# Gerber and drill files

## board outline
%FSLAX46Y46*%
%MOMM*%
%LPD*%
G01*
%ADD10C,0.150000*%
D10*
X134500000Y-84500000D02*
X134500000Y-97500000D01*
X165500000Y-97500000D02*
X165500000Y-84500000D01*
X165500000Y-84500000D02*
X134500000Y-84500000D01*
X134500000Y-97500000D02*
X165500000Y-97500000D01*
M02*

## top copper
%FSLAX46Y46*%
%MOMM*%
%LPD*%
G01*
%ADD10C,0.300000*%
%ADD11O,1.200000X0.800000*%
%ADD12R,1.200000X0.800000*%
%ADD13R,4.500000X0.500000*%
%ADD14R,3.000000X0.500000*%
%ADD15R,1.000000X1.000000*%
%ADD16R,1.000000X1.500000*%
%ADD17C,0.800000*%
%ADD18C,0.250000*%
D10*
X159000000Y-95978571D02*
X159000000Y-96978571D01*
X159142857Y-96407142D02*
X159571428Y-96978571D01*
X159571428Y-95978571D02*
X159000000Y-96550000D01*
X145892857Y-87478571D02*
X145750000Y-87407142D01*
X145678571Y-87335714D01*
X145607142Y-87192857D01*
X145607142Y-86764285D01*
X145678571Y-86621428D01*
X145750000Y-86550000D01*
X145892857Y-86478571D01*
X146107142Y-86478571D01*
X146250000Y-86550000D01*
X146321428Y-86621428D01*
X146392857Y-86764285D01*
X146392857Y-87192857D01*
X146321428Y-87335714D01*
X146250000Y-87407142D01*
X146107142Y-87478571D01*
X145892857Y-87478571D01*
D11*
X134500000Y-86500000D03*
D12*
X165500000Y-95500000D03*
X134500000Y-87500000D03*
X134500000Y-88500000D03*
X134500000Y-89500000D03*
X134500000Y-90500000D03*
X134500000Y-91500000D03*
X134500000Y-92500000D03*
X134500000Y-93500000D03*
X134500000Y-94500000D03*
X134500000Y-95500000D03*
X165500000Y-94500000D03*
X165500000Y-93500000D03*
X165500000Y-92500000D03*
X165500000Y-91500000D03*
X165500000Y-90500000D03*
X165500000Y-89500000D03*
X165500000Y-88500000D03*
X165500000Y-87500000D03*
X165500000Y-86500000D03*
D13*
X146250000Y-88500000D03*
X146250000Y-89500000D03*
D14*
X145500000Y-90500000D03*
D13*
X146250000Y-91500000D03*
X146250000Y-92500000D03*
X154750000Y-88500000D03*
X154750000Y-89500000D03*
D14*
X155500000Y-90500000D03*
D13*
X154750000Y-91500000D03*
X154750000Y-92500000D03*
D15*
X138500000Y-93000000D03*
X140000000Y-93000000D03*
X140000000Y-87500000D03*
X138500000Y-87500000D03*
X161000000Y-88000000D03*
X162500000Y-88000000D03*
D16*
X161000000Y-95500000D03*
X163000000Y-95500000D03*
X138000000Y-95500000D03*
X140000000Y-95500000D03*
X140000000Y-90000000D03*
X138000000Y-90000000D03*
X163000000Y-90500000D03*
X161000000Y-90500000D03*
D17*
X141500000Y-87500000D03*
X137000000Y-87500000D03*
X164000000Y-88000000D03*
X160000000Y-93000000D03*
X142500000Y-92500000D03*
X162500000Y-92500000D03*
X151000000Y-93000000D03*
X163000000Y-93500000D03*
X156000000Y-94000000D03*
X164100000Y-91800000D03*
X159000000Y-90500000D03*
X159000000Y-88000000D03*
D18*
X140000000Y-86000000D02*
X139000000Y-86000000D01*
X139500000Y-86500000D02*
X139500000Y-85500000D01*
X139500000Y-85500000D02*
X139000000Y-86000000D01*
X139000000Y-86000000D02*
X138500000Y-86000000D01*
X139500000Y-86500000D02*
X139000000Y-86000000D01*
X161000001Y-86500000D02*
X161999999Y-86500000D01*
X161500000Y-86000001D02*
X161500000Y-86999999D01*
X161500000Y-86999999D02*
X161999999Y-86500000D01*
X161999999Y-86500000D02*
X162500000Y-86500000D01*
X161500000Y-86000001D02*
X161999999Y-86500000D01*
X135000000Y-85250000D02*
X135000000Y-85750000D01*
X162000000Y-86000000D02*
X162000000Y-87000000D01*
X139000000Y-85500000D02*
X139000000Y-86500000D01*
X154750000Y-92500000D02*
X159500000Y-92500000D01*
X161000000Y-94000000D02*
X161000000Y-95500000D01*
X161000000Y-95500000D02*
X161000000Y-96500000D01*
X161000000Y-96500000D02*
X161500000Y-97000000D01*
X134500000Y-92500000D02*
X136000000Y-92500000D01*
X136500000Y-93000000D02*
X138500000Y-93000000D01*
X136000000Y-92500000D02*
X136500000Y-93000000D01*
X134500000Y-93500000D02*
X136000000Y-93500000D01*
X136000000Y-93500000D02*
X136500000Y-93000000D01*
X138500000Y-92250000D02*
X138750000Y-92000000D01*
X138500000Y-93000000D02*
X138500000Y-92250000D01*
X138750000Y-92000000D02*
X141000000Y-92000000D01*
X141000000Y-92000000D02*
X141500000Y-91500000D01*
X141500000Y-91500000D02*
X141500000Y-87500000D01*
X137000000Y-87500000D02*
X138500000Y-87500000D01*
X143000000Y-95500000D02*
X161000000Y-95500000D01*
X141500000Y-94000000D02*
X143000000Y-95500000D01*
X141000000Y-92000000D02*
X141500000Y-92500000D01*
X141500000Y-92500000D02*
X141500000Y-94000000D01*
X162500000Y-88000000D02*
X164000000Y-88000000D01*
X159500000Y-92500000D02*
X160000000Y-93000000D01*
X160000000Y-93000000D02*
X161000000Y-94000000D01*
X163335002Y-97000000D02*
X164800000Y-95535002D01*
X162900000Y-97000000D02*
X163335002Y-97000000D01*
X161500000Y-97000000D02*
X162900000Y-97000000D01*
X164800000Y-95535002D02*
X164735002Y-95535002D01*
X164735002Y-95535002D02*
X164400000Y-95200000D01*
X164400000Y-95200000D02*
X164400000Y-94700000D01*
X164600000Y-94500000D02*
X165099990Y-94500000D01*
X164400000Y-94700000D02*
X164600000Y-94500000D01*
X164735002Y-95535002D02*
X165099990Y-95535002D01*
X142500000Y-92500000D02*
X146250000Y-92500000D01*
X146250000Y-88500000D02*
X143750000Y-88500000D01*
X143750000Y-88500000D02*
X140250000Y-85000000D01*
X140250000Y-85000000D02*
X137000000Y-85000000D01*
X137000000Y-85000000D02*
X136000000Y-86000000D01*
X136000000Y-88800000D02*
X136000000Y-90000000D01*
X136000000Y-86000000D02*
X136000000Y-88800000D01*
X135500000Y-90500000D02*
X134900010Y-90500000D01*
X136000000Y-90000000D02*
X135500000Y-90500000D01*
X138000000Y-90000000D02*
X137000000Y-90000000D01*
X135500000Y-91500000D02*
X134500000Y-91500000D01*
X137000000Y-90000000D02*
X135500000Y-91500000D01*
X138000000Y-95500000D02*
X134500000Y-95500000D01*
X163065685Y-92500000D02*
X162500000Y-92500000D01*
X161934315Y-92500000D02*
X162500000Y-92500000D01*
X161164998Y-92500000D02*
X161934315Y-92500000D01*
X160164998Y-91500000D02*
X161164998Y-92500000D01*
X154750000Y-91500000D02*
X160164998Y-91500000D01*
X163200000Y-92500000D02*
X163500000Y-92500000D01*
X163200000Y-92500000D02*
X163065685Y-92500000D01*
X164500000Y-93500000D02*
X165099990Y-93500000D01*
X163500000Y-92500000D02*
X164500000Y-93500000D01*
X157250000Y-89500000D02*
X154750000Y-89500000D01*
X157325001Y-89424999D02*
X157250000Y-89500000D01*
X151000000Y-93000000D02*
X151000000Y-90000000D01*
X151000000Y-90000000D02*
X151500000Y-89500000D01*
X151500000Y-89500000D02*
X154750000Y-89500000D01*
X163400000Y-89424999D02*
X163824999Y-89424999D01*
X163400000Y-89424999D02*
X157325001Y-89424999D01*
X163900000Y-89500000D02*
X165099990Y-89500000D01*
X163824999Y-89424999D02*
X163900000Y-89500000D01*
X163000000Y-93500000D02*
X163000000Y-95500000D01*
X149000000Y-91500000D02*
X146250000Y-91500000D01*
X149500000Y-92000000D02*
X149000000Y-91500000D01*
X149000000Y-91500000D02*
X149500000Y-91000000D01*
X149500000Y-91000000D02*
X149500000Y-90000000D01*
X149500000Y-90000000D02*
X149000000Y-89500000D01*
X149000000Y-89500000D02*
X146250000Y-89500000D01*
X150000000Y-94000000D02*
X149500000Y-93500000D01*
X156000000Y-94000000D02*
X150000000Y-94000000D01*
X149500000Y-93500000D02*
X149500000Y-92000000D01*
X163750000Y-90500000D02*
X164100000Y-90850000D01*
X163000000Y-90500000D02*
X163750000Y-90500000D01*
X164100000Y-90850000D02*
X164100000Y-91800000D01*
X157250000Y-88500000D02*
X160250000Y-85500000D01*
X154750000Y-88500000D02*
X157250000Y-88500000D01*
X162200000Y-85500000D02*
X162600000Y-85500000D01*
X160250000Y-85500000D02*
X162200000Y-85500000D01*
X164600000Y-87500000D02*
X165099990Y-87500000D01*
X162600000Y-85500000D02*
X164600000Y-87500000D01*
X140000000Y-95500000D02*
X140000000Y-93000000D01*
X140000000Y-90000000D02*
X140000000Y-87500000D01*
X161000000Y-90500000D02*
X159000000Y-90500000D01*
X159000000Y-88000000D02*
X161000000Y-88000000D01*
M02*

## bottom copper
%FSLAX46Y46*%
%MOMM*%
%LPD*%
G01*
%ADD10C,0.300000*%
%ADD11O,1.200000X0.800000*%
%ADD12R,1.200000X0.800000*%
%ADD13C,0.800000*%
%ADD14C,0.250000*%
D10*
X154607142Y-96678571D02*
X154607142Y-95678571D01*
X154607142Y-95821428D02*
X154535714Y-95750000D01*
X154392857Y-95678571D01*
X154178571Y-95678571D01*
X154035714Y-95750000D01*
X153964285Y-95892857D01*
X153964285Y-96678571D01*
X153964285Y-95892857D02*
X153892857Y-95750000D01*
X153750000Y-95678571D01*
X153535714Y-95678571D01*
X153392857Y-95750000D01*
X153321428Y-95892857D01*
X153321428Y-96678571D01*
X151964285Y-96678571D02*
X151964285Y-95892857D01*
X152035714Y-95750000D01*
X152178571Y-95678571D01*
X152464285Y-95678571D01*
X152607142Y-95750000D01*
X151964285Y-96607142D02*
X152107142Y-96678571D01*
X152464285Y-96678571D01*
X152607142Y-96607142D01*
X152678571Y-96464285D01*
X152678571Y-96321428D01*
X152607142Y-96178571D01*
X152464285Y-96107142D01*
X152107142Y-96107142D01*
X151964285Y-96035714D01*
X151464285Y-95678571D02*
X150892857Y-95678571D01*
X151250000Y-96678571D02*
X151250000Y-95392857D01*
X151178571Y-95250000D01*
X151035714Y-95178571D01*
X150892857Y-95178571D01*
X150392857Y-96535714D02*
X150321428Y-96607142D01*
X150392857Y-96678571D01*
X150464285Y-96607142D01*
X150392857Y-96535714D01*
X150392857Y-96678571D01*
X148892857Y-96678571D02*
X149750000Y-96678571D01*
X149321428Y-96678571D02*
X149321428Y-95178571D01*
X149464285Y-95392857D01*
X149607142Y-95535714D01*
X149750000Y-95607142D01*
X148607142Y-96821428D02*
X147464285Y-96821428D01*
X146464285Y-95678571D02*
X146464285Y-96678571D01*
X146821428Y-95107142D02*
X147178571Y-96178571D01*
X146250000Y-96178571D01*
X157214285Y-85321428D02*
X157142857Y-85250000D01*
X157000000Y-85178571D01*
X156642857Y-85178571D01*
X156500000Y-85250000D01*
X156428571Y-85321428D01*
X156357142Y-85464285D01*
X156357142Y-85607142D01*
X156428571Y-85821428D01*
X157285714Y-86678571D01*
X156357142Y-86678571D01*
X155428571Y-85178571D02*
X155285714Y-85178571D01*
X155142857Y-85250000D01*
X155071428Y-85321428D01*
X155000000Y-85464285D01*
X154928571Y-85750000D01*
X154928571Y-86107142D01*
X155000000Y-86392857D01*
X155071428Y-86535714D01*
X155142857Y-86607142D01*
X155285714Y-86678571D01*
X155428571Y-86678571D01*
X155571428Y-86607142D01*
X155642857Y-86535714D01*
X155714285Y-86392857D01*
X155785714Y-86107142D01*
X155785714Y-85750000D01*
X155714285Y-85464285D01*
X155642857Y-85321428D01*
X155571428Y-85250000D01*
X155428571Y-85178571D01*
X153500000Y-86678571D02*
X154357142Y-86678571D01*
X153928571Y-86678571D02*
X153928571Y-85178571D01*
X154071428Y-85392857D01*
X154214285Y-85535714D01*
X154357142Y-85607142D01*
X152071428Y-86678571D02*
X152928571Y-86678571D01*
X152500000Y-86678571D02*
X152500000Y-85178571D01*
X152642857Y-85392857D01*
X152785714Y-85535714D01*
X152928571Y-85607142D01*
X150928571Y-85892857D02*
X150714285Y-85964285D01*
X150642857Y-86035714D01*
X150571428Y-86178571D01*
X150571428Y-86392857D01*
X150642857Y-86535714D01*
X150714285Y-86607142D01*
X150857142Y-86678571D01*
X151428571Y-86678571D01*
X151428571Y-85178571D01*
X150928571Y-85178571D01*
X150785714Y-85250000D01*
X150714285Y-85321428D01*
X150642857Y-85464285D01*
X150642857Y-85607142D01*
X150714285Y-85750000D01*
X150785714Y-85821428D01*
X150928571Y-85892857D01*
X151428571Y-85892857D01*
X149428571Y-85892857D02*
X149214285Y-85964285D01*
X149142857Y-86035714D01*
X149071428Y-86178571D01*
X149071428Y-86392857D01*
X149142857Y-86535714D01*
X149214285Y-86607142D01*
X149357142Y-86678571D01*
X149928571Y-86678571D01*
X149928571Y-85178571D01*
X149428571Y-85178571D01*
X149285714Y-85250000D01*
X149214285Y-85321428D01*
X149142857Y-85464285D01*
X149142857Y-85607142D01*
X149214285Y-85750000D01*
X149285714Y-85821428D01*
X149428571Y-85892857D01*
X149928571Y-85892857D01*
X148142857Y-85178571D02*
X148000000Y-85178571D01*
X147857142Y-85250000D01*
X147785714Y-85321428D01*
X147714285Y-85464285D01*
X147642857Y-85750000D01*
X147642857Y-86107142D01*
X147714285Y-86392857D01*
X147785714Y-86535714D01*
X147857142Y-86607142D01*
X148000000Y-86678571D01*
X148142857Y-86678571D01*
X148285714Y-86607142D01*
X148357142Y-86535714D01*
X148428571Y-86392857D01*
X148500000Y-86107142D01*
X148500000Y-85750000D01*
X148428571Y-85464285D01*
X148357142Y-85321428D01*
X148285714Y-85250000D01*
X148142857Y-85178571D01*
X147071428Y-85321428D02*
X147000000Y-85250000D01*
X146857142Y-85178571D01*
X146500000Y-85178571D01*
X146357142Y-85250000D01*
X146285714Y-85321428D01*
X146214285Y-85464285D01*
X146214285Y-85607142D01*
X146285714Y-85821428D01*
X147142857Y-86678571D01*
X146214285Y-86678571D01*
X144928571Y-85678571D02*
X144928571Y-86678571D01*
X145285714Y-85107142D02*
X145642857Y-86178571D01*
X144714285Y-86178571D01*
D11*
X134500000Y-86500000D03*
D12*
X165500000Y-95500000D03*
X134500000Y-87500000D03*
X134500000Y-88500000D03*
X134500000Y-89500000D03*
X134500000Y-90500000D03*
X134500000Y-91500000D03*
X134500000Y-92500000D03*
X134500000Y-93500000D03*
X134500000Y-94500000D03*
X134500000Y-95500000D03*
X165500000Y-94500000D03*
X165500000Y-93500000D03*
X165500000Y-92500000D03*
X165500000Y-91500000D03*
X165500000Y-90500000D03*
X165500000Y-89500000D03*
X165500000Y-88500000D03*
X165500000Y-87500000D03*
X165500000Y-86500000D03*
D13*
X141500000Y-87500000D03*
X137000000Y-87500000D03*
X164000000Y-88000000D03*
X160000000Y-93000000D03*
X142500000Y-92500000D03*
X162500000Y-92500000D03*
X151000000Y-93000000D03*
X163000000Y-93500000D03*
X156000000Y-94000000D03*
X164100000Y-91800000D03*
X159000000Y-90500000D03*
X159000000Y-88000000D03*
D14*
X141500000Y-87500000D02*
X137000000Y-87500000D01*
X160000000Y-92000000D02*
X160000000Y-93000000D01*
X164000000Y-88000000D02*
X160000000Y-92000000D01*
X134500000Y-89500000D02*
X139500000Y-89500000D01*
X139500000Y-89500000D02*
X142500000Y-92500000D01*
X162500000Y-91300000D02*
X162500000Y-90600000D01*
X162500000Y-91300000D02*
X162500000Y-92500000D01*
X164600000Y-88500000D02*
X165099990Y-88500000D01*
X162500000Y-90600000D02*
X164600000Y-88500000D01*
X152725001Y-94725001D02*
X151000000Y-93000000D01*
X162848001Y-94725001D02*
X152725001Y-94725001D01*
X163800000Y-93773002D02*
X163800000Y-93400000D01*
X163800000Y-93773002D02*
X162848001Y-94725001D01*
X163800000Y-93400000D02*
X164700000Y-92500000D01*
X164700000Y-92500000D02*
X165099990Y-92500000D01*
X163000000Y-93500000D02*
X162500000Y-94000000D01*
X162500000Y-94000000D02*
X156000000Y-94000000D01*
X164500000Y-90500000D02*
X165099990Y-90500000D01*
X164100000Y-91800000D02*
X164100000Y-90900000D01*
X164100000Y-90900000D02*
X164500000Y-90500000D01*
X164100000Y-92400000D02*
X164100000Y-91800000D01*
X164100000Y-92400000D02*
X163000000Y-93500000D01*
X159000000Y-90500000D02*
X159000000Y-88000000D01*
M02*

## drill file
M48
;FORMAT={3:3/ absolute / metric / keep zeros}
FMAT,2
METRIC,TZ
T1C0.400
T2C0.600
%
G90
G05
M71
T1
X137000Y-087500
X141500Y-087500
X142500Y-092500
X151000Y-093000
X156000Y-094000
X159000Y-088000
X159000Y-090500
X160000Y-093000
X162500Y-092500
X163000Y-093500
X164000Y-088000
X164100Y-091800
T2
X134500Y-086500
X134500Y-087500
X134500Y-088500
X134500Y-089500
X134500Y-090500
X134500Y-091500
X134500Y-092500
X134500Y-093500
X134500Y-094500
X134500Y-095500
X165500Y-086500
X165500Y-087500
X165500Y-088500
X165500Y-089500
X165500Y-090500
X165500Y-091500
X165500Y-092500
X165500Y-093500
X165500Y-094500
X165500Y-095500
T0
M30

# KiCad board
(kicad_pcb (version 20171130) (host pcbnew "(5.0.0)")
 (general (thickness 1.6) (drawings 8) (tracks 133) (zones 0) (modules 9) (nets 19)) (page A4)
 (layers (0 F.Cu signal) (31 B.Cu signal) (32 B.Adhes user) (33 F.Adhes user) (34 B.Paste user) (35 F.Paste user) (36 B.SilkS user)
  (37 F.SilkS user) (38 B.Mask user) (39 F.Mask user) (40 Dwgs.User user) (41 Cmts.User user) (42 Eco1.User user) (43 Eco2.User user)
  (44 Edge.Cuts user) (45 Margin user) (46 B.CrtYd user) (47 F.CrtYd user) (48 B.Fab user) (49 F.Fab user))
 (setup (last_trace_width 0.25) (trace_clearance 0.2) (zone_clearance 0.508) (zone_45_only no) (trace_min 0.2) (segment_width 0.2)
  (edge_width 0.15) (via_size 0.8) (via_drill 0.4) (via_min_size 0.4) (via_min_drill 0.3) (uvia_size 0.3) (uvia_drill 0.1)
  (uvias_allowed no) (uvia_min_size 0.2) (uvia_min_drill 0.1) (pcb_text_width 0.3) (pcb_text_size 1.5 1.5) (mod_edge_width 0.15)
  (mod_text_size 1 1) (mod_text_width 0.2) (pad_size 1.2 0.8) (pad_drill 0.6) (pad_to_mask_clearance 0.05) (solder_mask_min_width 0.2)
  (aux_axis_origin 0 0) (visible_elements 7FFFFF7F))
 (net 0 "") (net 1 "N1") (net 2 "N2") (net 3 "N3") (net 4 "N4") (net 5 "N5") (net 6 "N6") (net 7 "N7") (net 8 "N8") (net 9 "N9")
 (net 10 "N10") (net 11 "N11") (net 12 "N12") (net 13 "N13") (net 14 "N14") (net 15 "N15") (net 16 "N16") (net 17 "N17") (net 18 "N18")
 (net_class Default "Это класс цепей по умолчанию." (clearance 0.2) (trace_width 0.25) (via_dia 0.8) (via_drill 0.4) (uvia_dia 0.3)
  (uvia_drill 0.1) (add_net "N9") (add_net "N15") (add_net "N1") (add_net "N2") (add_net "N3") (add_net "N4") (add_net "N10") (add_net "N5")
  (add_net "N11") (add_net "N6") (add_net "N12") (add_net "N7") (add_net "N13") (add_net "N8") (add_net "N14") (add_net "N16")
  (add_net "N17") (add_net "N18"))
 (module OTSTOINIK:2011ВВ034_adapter (layer F.Cu) (at 150 91)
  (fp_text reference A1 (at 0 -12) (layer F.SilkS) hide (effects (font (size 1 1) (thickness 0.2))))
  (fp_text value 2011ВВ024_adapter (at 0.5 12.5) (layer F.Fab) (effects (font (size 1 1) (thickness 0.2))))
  (pad 1A thru_hole oval (at -15.5 -4.5) (size 1.2 0.8) (drill 0.6) (layers *.Cu *.Mask) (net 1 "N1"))
  (pad 1B thru_hole rect (at 15.5 4.5) (size 1.2 0.8) (drill 0.6) (layers *.Cu *.Mask) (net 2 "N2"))
  (pad 2A thru_hole rect (at -15.5 -3.5) (size 1.2 0.8) (drill 0.6) (layers *.Cu *.Mask) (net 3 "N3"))
  (pad 3A thru_hole rect (at -15.5 -2.5) (size 1.2 0.8) (drill 0.6) (layers *.Cu *.Mask) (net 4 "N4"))
  (pad 4A thru_hole rect (at -15.5 -1.5) (size 1.2 0.8) (drill 0.6) (layers *.Cu *.Mask) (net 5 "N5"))
  (pad 5A thru_hole rect (at -15.5 -0.5) (size 1.2 0.8) (drill 0.6) (layers *.Cu *.Mask) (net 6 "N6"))
  (pad 6A thru_hole rect (at -15.5 0.5) (size 1.2 0.8) (drill 0.6) (layers *.Cu *.Mask) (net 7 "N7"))
  (pad 7A thru_hole rect (at -15.5 1.5) (size 1.2 0.8) (drill 0.6) (layers *.Cu *.Mask) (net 2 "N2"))
  (pad 8A thru_hole rect (at -15.5 2.5) (size 1.2 0.8) (drill 0.6) (layers *.Cu *.Mask) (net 2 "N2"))
  (pad 9A thru_hole rect (at -15.5 3.5) (size 1.2 0.8) (drill 0.6) (layers *.Cu *.Mask) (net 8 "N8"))
  (pad 10A thru_hole rect (at -15.5 4.5) (size 1.2 0.8) (drill 0.6) (layers *.Cu *.Mask) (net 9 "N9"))
  (pad 2B thru_hole rect (at 15.5 3.5) (size 1.2 0.8) (drill 0.6) (layers *.Cu *.Mask) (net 2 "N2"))
  (pad 3B thru_hole rect (at 15.5 2.5) (size 1.2 0.8) (drill 0.6) (layers *.Cu *.Mask) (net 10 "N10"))
  (pad 4B thru_hole rect (at 15.5 1.5) (size 1.2 0.8) (drill 0.6) (layers *.Cu *.Mask) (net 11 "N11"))
  (pad 5B thru_hole rect (at 15.5 0.5) (size 1.2 0.8) (drill 0.6) (layers *.Cu *.Mask) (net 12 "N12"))
  (pad 6B thru_hole rect (at 15.5 -0.5) (size 1.2 0.8) (drill 0.6) (layers *.Cu *.Mask) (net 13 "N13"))
  (pad 7B thru_hole rect (at 15.5 -1.5) (size 1.2 0.8) (drill 0.6) (layers *.Cu *.Mask) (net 11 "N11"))
  (pad 8B thru_hole rect (at 15.5 -2.5) (size 1.2 0.8) (drill 0.6) (layers *.Cu *.Mask) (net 10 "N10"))
  (pad 9B thru_hole rect (at 15.5 -3.5) (size 1.2 0.8) (drill 0.6) (layers *.Cu *.Mask) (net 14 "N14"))
  (pad 10B thru_hole rect (at 15.5 -4.5) (size 1.2 0.8) (drill 0.6) (layers *.Cu *.Mask) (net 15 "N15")))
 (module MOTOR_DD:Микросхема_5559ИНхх (layer F.Cu) (at 148.5 94)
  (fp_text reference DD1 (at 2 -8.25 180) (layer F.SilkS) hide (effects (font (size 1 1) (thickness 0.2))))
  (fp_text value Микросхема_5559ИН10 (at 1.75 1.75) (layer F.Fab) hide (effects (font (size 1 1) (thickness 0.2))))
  (pad 1 smd rect (at -2.25 -5.5) (size 4.5 0.5) (layers F.Cu F.Paste F.Mask) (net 6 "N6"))
  (pad 2 smd rect (at -2.25 -4.5) (size 4.5 0.5) (layers F.Cu F.Paste F.Mask) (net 13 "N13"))
  (pad "" smd rect (at -3 -3.5) (size 3 0.5) (layers F.Cu F.Paste F.Mask))
  (pad 3 smd rect (at -2.25 -2.5) (size 4.5 0.5) (layers F.Cu F.Paste F.Mask) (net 13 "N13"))
  (pad 4 smd rect (at -2.25 -1.5) (size 4.5 0.5) (layers F.Cu F.Paste F.Mask) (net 5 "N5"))
  (pad 8 smd rect (at 6.25 -5.5) (size 4.5 0.5) (layers F.Cu F.Paste F.Mask) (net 14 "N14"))
  (pad 7 smd rect (at 6.25 -4.5) (size 4.5 0.5) (layers F.Cu F.Paste F.Mask) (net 11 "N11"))
  (pad "" smd rect (at 7 -3.5) (size 3 0.5) (layers F.Cu F.Paste F.Mask))
  (pad 6 smd rect (at 6.25 -2.5) (size 4.5 0.5) (layers F.Cu F.Paste F.Mask) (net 10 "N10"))
  (pad 5 smd rect (at 6.25 -1.5) (size 4.5 0.5) (layers F.Cu F.Paste F.Mask) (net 2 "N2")))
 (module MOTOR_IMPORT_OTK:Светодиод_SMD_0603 (layer F.Cu) (at 140 93 180)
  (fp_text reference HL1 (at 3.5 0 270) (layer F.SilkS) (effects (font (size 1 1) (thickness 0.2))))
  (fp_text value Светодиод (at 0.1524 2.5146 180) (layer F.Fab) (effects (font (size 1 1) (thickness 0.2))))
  (pad 2 smd rect (at 1.5 0 180) (size 1 1) (layers F.Cu F.Paste F.Mask) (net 2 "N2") (clearance 0.2))
  (pad 1 smd rect (at 0 0 180) (size 1 1) (layers F.Cu F.Paste F.Mask) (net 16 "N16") (clearance 0.2)))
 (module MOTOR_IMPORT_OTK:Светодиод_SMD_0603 (layer F.Cu) (at 140 87.5 180)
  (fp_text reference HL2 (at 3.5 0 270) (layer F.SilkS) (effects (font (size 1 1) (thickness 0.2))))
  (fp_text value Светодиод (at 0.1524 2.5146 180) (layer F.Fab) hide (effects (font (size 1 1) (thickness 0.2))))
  (pad 1 smd rect (at 0 0 180) (size 1 1) (layers F.Cu F.Paste F.Mask) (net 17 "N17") (clearance 0.2))
  (pad 2 smd rect (at 1.5 0 180) (size 1 1) (layers F.Cu F.Paste F.Mask) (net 2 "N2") (clearance 0.2)))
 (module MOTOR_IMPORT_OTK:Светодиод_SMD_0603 (layer F.Cu) (at 161 88)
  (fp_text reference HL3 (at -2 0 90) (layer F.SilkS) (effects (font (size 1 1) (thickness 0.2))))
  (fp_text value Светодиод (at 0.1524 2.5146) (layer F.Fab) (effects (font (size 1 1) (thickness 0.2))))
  (pad 1 smd rect (at 0 0) (size 1 1) (layers F.Cu F.Paste F.Mask) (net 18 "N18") (clearance 0.2))
  (pad 2 smd rect (at 1.5 0) (size 1 1) (layers F.Cu F.Paste F.Mask) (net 2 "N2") (clearance 0.2)))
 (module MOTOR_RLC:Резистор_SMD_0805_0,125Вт (layer F.Cu) (at 163 95.5 180)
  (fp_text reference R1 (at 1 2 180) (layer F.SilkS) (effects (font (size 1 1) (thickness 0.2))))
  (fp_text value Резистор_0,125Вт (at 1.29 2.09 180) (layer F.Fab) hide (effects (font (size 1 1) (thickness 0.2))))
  (pad 2 smd rect (at 2 0 180) (size 1 1.5) (layers F.Cu F.Paste F.Mask) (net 2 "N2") (clearance 0.2))
  (pad 1 smd rect (at 0 0 180) (size 1 1.5) (layers F.Cu F.Paste F.Mask) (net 13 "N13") (clearance 0.2)))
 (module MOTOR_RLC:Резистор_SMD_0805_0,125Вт (layer F.Cu) (at 140 95.5 180)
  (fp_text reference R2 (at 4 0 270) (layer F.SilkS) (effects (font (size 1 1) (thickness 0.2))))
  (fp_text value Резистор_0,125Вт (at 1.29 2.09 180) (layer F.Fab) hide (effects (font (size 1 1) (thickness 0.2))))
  (pad 2 smd rect (at 2 0 180) (size 1 1.5) (layers F.Cu F.Paste F.Mask) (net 9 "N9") (clearance 0.2))
  (pad 1 smd rect (at 0 0 180) (size 1 1.5) (layers F.Cu F.Paste F.Mask) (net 16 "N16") (clearance 0.2)))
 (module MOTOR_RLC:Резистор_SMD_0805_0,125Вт (layer F.Cu) (at 140 90 180)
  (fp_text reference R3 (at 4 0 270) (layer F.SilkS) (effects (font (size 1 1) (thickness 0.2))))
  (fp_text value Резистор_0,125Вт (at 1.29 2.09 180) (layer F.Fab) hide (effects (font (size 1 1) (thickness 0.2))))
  (pad 1 smd rect (at 0 0 180) (size 1 1.5) (layers F.Cu F.Paste F.Mask) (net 17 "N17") (clearance 0.2))
  (pad 2 smd rect (at 2 0 180) (size 1 1.5) (layers F.Cu F.Paste F.Mask) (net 7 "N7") (clearance 0.2)))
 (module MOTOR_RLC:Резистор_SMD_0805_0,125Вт (layer F.Cu) (at 163 90.5 180)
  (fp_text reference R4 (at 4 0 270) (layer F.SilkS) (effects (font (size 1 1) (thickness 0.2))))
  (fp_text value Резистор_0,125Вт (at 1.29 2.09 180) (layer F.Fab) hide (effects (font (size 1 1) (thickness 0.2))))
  (pad 1 smd rect (at 0 0 180) (size 1 1.5) (layers F.Cu F.Paste F.Mask) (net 13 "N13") (clearance 0.2))
  (pad 2 smd rect (at 2 0 180) (size 1 1.5) (layers F.Cu F.Paste F.Mask) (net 18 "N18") (clearance 0.2)))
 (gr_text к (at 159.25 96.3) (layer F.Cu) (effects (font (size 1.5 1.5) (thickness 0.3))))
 (gr_line (start 134.5 84.5) (end 134.5 97.5) (layer Edge.Cuts) (width 0.15))
 (gr_line (start 165.5 97.5) (end 165.5 84.5) (layer Edge.Cuts) (width 0.15))
 (gr_line (start 165.5 84.5) (end 134.5 84.5) (layer Edge.Cuts) (width 0.15))
 (gr_line (start 134.5 97.5) (end 165.5 97.5) (layer Edge.Cuts) (width 0.15))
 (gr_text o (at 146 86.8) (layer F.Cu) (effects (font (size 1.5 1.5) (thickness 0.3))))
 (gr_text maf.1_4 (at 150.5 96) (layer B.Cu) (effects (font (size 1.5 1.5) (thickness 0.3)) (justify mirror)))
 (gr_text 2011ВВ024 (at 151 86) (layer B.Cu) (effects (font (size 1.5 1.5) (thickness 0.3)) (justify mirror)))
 (segment (start 140 86) (end 139 86) (width 0.25) (layer F.Cu) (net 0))
 (segment (start 139.5 86.5) (end 139.5 85.5) (width 0.25) (layer F.Cu) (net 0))
 (segment (start 139.5 85.5) (end 139 86) (width 0.25) (layer F.Cu) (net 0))
 (segment (start 139 86) (end 138.5 86) (width 0.25) (layer F.Cu) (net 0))
 (segment (start 139.5 86.5) (end 139 86) (width 0.25) (layer F.Cu) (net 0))
 (segment (start 161.000001 86.5) (end 161.999999 86.5) (width 0.25) (layer F.Cu) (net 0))
 (segment (start 161.5 86.000001) (end 161.5 86.999999) (width 0.25) (layer F.Cu) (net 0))
 (segment (start 161.5 86.999999) (end 161.999999 86.5) (width 0.25) (layer F.Cu) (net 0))
 (segment (start 161.999999 86.5) (end 162.5 86.5) (width 0.25) (layer F.Cu) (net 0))
 (segment (start 161.5 86.000001) (end 161.999999 86.5) (width 0.25) (layer F.Cu) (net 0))
 (segment (start 135 85.25) (end 135 85.75) (width 0.25) (layer F.Cu) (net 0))
 (segment (start 162 86) (end 162 87) (width 0.25) (layer F.Cu) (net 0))
 (segment (start 139 85.5) (end 139 86.5) (width 0.25) (layer F.Cu) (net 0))
 (segment (start 154.75 92.5) (end 159.5 92.5) (width 0.25) (layer F.Cu) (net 2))
 (segment (start 161 94) (end 161 95.5) (width 0.25) (layer F.Cu) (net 2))
 (segment (start 161 95.5) (end 161 96.5) (width 0.25) (layer F.Cu) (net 2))
 (segment (start 161 96.5) (end 161.5 97) (width 0.25) (layer F.Cu) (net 2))
 (segment (start 134.5 92.5) (end 136 92.5) (width 0.25) (layer F.Cu) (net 2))
 (segment (start 136.5 93) (end 138.5 93) (width 0.25) (layer F.Cu) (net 2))
 (segment (start 136 92.5) (end 136.5 93) (width 0.25) (layer F.Cu) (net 2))
 (segment (start 134.5 93.5) (end 136 93.5) (width 0.25) (layer F.Cu) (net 2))
 (segment (start 136 93.5) (end 136.5 93) (width 0.25) (layer F.Cu) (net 2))
 (segment (start 138.5 92.25) (end 138.75 92) (width 0.25) (layer F.Cu) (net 2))
 (segment (start 138.5 93) (end 138.5 92.25) (width 0.25) (layer F.Cu) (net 2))
 (segment (start 138.75 92) (end 141 92) (width 0.25) (layer F.Cu) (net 2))
 (via (at 141.5 87.5) (size 0.8) (drill 0.4) (layers F.Cu B.Cu) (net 2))
 (segment (start 141 92) (end 141.5 91.5) (width 0.25) (layer F.Cu) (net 2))
 (segment (start 141.5 91.5) (end 141.5 87.5) (width 0.25) (layer F.Cu) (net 2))
 (via (at 137 87.5) (size 0.8) (drill 0.4) (layers F.Cu B.Cu) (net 2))
 (segment (start 141.5 87.5) (end 137 87.5) (width 0.25) (layer B.Cu) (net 2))
 (segment (start 137 87.5) (end 138.5 87.5) (width 0.25) (layer F.Cu) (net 2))
 (segment (start 143 95.5) (end 161 95.5) (width 0.25) (layer F.Cu) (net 2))
 (segment (start 141.5 94) (end 143 95.5) (width 0.25) (layer F.Cu) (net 2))
 (segment (start 141 92) (end 141.5 92.5) (width 0.25) (layer F.Cu) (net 2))
 (segment (start 141.5 92.5) (end 141.5 94) (width 0.25) (layer F.Cu) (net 2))
 (via (at 164 88) (size 0.8) (drill 0.4) (layers F.Cu B.Cu) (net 2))
 (segment (start 162.5 88) (end 164 88) (width 0.25) (layer F.Cu) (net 2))
 (via (at 160 93) (size 0.8) (drill 0.4) (layers F.Cu B.Cu) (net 2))
 (segment (start 160 92) (end 160 93) (width 0.25) (layer B.Cu) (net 2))
 (segment (start 164 88) (end 160 92) (width 0.25) (layer B.Cu) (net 2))
 (segment (start 159.5 92.5) (end 160 93) (width 0.25) (layer F.Cu) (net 2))
 (segment (start 160 93) (end 161 94) (width 0.25) (layer F.Cu) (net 2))
 (segment (start 163.335002 97) (end 164.8 95.535002) (width 0.25) (layer F.Cu) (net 2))
 (segment (start 162.9 97) (end 163.335002 97) (width 0.25) (layer F.Cu) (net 2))
 (segment (start 161.5 97) (end 162.9 97) (width 0.25) (layer F.Cu) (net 2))
 (segment (start 164.8 95.535002) (end 164.735002 95.535002) (width 0.25) (layer F.Cu) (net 2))
 (segment (start 164.735002 95.535002) (end 164.4 95.2) (width 0.25) (layer F.Cu) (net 2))
 (segment (start 164.4 95.2) (end 164.4 94.7) (width 0.25) (layer F.Cu) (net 2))
 (segment (start 164.6 94.5) (end 165.09999 94.5) (width 0.25) (layer F.Cu) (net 2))
 (segment (start 164.4 94.7) (end 164.6 94.5) (width 0.25) (layer F.Cu) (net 2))
 (segment (start 164.735002 95.535002) (end 165.09999 95.535002) (width 0.25) (layer F.Cu) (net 2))
 (via (at 142.5 92.5) (size 0.8) (drill 0.4) (layers F.Cu B.Cu) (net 5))
 (segment (start 134.5 89.5) (end 139.5 89.5) (width 0.25) (layer B.Cu) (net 5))
 (segment (start 139.5 89.5) (end 142.5 92.5) (width 0.25) (layer B.Cu) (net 5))
 (segment (start 142.5 92.5) (end 146.25 92.5) (width 0.25) (layer F.Cu) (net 5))
 (segment (start 146.25 88.5) (end 143.75 88.5) (width 0.25) (layer F.Cu) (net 6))
 (segment (start 143.75 88.5) (end 140.25 85) (width 0.25) (layer F.Cu) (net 6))
 (segment (start 140.25 85) (end 137 85) (width 0.25) (layer F.Cu) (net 6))
 (segment (start 137 85) (end 136 86) (width 0.25) (layer F.Cu) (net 6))
 (segment (start 136 88.8) (end 136 90) (width 0.25) (layer F.Cu) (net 6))
 (segment (start 136 86) (end 136 88.8) (width 0.25) (layer F.Cu) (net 6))
 (segment (start 135.5 90.5) (end 134.90001 90.5) (width 0.25) (layer F.Cu) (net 6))
 (segment (start 136 90) (end 135.5 90.5) (width 0.25) (layer F.Cu) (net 6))
 (segment (start 138 90) (end 137 90) (width 0.25) (layer F.Cu) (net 7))
 (segment (start 135.5 91.5) (end 134.5 91.5) (width 0.25) (layer F.Cu) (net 7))
 (segment (start 137 90) (end 135.5 91.5) (width 0.25) (layer F.Cu) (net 7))
 (segment (start 138 95.5) (end 134.5 95.5) (width 0.25) (layer F.Cu) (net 9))
 (via (at 162.5 92.5) (size 0.8) (drill 0.4) (layers F.Cu B.Cu) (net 10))
 (segment (start 163.065685 92.5) (end 162.5 92.5) (width 0.25) (layer F.Cu) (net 10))
 (segment (start 161.934315 92.5) (end 162.5 92.5) (width 0.25) (layer F.Cu) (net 10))
 (segment (start 161.164998 92.5) (end 161.934315 92.5) (width 0.25) (layer F.Cu) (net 10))
 (segment (start 160.164998 91.5) (end 161.164998 92.5) (width 0.25) (layer F.Cu) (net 10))
 (segment (start 154.75 91.5) (end 160.164998 91.5) (width 0.25) (layer F.Cu) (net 10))
 (segment (start 163.2 92.5) (end 163.5 92.5) (width 0.25) (layer F.Cu) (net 10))
 (segment (start 163.2 92.5) (end 163.065685 92.5) (width 0.25) (layer F.Cu) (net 10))
 (segment (start 164.5 93.5) (end 165.09999 93.5) (width 0.25) (layer F.Cu) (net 10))
 (segment (start 163.5 92.5) (end 164.5 93.5) (width 0.25) (layer F.Cu) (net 10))
 (segment (start 162.5 91.3) (end 162.5 90.6) (width 0.25) (layer B.Cu) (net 10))
 (segment (start 162.5 91.3) (end 162.5 92.5) (width 0.25) (layer B.Cu) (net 10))
 (segment (start 164.6 88.5) (end 165.09999 88.5) (width 0.25) (layer B.Cu) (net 10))
 (segment (start 162.5 90.6) (end 164.6 88.5) (width 0.25) (layer B.Cu) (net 10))
 (segment (start 157.25 89.5) (end 154.75 89.5) (width 0.25) (layer F.Cu) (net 11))
 (segment (start 157.325001 89.424999) (end 157.25 89.5) (width 0.25) (layer F.Cu) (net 11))
 (via (at 151 93) (size 0.8) (drill 0.4) (layers F.Cu B.Cu) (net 11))
 (segment (start 152.725001 94.725001) (end 151 93) (width 0.25) (layer B.Cu) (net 11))
 (segment (start 162.848001 94.725001) (end 152.725001 94.725001) (width 0.25) (layer B.Cu) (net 11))
 (segment (start 151 93) (end 151 90) (width 0.25) (layer F.Cu) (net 11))
 (segment (start 151 90) (end 151.5 89.5) (width 0.25) (layer F.Cu) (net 11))
 (segment (start 151.5 89.5) (end 154.75 89.5) (width 0.25) (layer F.Cu) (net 11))
 (segment (start 163.8 93.773002) (end 163.8 93.4) (width 0.25) (layer B.Cu) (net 11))
 (segment (start 163.8 93.773002) (end 162.848001 94.725001) (width 0.25) (layer B.Cu) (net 11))
 (segment (start 163.8 93.4) (end 164.7 92.5) (width 0.25) (layer B.Cu) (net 11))
 (segment (start 164.7 92.5) (end 165.09999 92.5) (width 0.25) (layer B.Cu) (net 11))
 (segment (start 163.4 89.424999) (end 163.824999 89.424999) (width 0.25) (layer F.Cu) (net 11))
 (segment (start 163.4 89.424999) (end 157.325001 89.424999) (width 0.25) (layer F.Cu) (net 11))
 (segment (start 163.9 89.5) (end 165.09999 89.5) (width 0.25) (layer F.Cu) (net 11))
 (segment (start 163.824999 89.424999) (end 163.9 89.5) (width 0.25) (layer F.Cu) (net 11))
 (via (at 163 93.5) (size 0.8) (drill 0.4) (layers F.Cu B.Cu) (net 13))
 (segment (start 163 93.5) (end 163 95.5) (width 0.25) (layer F.Cu) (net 13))
 (segment (start 163 93.5) (end 162.5 94) (width 0.25) (layer B.Cu) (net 13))
 (segment (start 162.5 94) (end 156 94) (width 0.25) (layer B.Cu) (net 13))
 (segment (start 149 91.5) (end 146.25 91.5) (width 0.25) (layer F.Cu) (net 13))
 (segment (start 149.5 92) (end 149 91.5) (width 0.25) (layer F.Cu) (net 13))
 (segment (start 149 91.5) (end 149.5 91) (width 0.25) (layer F.Cu) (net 13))
 (segment (start 149.5 91) (end 149.5 90) (width 0.25) (layer F.Cu) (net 13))
 (segment (start 149.5 90) (end 149 89.5) (width 0.25) (layer F.Cu) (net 13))
 (segment (start 149 89.5) (end 146.25 89.5) (width 0.25) (layer F.Cu) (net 13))
 (via (at 156 94) (size 0.8) (drill 0.4) (layers F.Cu B.Cu) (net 13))
 (segment (start 150 94) (end 149.5 93.5) (width 0.25) (layer F.Cu) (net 13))
 (segment (start 156 94) (end 150 94) (width 0.25) (layer F.Cu) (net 13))
 (segment (start 149.5 93.5) (end 149.5 92) (width 0.25) (layer F.Cu) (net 13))
 (via (at 164.1 91.8) (size 0.8) (drill 0.4) (layers F.Cu B.Cu) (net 13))
 (segment (start 164.5 90.5) (end 165.09999 90.5) (width 0.25) (layer B.Cu) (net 13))
 (segment (start 164.1 91.8) (end 164.1 90.9) (width 0.25) (layer B.Cu) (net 13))
 (segment (start 164.1 90.9) (end 164.5 90.5) (width 0.25) (layer B.Cu) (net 13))
 (segment (start 164.1 92.4) (end 164.1 91.8) (width 0.25) (layer B.Cu) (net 13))
 (segment (start 164.1 92.4) (end 163 93.5) (width 0.25) (layer B.Cu) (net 13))
 (segment (start 163.75 90.5) (end 164.1 90.85) (width 0.25) (layer F.Cu) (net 13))
 (segment (start 163 90.5) (end 163.75 90.5) (width 0.25) (layer F.Cu) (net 13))
 (segment (start 164.1 90.85) (end 164.1 91.8) (width 0.25) (layer F.Cu) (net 13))
 (segment (start 157.25 88.5) (end 160.25 85.5) (width 0.25) (layer F.Cu) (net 14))
 (segment (start 154.75 88.5) (end 157.25 88.5) (width 0.25) (layer F.Cu) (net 14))
 (segment (start 162.2 85.5) (end 162.6 85.5) (width 0.25) (layer F.Cu) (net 14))
 (segment (start 160.25 85.5) (end 162.2 85.5) (width 0.25) (layer F.Cu) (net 14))
 (segment (start 164.6 87.5) (end 165.09999 87.5) (width 0.25) (layer F.Cu) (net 14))
 (segment (start 162.6 85.5) (end 164.6 87.5) (width 0.25) (layer F.Cu) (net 14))
 (segment (start 140 95.5) (end 140 93) (width 0.25) (layer F.Cu) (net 16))
 (segment (start 140 90) (end 140 87.5) (width 0.25) (layer F.Cu) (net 17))
 (via (at 159 90.5) (size 0.8) (drill 0.4) (layers F.Cu B.Cu) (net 18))
 (segment (start 161 90.5) (end 159 90.5) (width 0.25) (layer F.Cu) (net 18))
 (via (at 159 88) (size 0.8) (drill 0.4) (layers F.Cu B.Cu) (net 18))
 (segment (start 159 90.5) (end 159 88) (width 0.25) (layer B.Cu) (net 18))
 (segment (start 159 88) (end 161 88) (width 0.25) (layer F.Cu) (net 18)))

